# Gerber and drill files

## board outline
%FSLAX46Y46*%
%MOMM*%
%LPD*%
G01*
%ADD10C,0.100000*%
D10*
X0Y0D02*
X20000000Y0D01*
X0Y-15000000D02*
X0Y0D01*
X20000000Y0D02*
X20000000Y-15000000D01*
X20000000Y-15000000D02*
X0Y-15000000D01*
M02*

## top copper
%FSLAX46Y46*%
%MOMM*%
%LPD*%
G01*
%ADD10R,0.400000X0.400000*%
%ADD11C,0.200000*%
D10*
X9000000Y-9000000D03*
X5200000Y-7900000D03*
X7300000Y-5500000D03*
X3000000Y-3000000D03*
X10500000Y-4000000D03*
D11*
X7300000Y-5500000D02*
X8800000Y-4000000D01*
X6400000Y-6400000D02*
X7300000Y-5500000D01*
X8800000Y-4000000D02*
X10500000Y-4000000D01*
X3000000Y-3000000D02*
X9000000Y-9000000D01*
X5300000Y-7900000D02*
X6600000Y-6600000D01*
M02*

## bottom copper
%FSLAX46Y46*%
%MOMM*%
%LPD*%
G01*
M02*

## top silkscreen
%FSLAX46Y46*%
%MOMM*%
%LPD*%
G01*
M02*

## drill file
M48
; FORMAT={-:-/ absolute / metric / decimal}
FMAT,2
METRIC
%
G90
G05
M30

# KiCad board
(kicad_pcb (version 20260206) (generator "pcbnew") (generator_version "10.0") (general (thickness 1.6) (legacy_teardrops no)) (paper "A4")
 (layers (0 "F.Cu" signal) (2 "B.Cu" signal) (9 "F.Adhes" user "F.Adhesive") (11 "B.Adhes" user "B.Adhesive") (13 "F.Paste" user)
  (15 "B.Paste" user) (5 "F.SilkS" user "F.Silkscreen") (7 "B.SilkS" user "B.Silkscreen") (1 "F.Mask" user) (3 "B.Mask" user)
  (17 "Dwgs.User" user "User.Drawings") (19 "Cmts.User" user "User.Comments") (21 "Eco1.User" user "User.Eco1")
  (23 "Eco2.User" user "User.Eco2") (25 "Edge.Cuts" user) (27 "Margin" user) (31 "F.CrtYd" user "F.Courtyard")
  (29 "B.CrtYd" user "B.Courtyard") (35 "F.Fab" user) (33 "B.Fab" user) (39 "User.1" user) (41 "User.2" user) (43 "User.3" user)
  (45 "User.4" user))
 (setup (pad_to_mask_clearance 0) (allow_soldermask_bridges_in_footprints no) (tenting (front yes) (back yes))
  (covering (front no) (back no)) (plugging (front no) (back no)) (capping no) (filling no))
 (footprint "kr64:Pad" (layer "F.Cu") (at 9 9)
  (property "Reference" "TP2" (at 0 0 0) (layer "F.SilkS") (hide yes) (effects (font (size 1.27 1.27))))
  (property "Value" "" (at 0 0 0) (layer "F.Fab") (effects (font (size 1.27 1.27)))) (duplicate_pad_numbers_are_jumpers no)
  (pad "1" smd rect (at 0 0) (size 0.4 0.4) (layers "F.Cu" "F.Mask" "F.Paste") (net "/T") (thermal_bridge_angle 45)))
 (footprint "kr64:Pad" (layer "F.Cu") (at 5.2 7.9)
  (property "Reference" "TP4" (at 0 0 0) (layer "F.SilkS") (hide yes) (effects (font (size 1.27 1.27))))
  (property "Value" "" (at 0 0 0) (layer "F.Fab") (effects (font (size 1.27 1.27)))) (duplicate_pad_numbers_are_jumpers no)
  (pad "1" smd rect (at 0 0) (size 0.4 0.4) (layers "F.Cu" "F.Mask" "F.Paste") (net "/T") (thermal_bridge_angle 45)))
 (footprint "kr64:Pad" (layer "F.Cu") (at 7.3 5.5)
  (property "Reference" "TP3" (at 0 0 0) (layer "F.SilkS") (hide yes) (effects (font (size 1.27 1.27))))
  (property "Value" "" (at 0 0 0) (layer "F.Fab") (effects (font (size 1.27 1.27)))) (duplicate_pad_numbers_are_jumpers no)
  (pad "1" smd rect (at 0 0) (size 0.4 0.4) (layers "F.Cu" "F.Mask" "F.Paste") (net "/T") (thermal_bridge_angle 45)))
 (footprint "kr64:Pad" (layer "F.Cu") (at 3 3)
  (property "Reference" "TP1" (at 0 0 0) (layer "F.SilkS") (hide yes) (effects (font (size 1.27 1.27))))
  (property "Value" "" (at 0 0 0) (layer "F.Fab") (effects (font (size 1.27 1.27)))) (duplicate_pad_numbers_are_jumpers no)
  (pad "1" smd rect (at 0 0) (size 0.4 0.4) (layers "F.Cu" "F.Mask" "F.Paste") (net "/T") (thermal_bridge_angle 45)))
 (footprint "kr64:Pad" (layer "F.Cu") (at 10.5 4)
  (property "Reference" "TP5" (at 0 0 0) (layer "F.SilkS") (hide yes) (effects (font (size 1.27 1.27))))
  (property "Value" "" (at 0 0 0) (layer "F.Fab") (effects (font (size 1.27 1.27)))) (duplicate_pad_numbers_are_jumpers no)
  (pad "1" smd rect (at 0 0) (size 0.4 0.4) (layers "F.Cu" "F.Mask" "F.Paste") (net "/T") (thermal_bridge_angle 45)))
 (gr_line (start 0 0) (end 20 0) (stroke (width 0.1) (type default)) (layer "Edge.Cuts"))
 (gr_line (start 0 15) (end 0 0) (stroke (width 0.1) (type default)) (layer "Edge.Cuts"))
 (gr_line (start 20 0) (end 20 15) (stroke (width 0.1) (type default)) (layer "Edge.Cuts"))
 (gr_line (start 20 15) (end 0 15) (stroke (width 0.1) (type default)) (layer "Edge.Cuts"))
 (segment (start 7.3 5.5) (end 8.8 4) (width 0.2) (layer "F.Cu") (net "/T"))
 (segment (start 6.4 6.4) (end 7.3 5.5) (width 0.2) (layer "F.Cu") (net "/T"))
 (segment (start 8.8 4) (end 10.5 4) (width 0.2) (layer "F.Cu") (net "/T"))
 (segment (start 3 3) (end 9 9) (width 0.2) (layer "F.Cu") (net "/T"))
 (segment (start 5.3 7.9) (end 6.6 6.6) (width 0.2) (layer "F.Cu") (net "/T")))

